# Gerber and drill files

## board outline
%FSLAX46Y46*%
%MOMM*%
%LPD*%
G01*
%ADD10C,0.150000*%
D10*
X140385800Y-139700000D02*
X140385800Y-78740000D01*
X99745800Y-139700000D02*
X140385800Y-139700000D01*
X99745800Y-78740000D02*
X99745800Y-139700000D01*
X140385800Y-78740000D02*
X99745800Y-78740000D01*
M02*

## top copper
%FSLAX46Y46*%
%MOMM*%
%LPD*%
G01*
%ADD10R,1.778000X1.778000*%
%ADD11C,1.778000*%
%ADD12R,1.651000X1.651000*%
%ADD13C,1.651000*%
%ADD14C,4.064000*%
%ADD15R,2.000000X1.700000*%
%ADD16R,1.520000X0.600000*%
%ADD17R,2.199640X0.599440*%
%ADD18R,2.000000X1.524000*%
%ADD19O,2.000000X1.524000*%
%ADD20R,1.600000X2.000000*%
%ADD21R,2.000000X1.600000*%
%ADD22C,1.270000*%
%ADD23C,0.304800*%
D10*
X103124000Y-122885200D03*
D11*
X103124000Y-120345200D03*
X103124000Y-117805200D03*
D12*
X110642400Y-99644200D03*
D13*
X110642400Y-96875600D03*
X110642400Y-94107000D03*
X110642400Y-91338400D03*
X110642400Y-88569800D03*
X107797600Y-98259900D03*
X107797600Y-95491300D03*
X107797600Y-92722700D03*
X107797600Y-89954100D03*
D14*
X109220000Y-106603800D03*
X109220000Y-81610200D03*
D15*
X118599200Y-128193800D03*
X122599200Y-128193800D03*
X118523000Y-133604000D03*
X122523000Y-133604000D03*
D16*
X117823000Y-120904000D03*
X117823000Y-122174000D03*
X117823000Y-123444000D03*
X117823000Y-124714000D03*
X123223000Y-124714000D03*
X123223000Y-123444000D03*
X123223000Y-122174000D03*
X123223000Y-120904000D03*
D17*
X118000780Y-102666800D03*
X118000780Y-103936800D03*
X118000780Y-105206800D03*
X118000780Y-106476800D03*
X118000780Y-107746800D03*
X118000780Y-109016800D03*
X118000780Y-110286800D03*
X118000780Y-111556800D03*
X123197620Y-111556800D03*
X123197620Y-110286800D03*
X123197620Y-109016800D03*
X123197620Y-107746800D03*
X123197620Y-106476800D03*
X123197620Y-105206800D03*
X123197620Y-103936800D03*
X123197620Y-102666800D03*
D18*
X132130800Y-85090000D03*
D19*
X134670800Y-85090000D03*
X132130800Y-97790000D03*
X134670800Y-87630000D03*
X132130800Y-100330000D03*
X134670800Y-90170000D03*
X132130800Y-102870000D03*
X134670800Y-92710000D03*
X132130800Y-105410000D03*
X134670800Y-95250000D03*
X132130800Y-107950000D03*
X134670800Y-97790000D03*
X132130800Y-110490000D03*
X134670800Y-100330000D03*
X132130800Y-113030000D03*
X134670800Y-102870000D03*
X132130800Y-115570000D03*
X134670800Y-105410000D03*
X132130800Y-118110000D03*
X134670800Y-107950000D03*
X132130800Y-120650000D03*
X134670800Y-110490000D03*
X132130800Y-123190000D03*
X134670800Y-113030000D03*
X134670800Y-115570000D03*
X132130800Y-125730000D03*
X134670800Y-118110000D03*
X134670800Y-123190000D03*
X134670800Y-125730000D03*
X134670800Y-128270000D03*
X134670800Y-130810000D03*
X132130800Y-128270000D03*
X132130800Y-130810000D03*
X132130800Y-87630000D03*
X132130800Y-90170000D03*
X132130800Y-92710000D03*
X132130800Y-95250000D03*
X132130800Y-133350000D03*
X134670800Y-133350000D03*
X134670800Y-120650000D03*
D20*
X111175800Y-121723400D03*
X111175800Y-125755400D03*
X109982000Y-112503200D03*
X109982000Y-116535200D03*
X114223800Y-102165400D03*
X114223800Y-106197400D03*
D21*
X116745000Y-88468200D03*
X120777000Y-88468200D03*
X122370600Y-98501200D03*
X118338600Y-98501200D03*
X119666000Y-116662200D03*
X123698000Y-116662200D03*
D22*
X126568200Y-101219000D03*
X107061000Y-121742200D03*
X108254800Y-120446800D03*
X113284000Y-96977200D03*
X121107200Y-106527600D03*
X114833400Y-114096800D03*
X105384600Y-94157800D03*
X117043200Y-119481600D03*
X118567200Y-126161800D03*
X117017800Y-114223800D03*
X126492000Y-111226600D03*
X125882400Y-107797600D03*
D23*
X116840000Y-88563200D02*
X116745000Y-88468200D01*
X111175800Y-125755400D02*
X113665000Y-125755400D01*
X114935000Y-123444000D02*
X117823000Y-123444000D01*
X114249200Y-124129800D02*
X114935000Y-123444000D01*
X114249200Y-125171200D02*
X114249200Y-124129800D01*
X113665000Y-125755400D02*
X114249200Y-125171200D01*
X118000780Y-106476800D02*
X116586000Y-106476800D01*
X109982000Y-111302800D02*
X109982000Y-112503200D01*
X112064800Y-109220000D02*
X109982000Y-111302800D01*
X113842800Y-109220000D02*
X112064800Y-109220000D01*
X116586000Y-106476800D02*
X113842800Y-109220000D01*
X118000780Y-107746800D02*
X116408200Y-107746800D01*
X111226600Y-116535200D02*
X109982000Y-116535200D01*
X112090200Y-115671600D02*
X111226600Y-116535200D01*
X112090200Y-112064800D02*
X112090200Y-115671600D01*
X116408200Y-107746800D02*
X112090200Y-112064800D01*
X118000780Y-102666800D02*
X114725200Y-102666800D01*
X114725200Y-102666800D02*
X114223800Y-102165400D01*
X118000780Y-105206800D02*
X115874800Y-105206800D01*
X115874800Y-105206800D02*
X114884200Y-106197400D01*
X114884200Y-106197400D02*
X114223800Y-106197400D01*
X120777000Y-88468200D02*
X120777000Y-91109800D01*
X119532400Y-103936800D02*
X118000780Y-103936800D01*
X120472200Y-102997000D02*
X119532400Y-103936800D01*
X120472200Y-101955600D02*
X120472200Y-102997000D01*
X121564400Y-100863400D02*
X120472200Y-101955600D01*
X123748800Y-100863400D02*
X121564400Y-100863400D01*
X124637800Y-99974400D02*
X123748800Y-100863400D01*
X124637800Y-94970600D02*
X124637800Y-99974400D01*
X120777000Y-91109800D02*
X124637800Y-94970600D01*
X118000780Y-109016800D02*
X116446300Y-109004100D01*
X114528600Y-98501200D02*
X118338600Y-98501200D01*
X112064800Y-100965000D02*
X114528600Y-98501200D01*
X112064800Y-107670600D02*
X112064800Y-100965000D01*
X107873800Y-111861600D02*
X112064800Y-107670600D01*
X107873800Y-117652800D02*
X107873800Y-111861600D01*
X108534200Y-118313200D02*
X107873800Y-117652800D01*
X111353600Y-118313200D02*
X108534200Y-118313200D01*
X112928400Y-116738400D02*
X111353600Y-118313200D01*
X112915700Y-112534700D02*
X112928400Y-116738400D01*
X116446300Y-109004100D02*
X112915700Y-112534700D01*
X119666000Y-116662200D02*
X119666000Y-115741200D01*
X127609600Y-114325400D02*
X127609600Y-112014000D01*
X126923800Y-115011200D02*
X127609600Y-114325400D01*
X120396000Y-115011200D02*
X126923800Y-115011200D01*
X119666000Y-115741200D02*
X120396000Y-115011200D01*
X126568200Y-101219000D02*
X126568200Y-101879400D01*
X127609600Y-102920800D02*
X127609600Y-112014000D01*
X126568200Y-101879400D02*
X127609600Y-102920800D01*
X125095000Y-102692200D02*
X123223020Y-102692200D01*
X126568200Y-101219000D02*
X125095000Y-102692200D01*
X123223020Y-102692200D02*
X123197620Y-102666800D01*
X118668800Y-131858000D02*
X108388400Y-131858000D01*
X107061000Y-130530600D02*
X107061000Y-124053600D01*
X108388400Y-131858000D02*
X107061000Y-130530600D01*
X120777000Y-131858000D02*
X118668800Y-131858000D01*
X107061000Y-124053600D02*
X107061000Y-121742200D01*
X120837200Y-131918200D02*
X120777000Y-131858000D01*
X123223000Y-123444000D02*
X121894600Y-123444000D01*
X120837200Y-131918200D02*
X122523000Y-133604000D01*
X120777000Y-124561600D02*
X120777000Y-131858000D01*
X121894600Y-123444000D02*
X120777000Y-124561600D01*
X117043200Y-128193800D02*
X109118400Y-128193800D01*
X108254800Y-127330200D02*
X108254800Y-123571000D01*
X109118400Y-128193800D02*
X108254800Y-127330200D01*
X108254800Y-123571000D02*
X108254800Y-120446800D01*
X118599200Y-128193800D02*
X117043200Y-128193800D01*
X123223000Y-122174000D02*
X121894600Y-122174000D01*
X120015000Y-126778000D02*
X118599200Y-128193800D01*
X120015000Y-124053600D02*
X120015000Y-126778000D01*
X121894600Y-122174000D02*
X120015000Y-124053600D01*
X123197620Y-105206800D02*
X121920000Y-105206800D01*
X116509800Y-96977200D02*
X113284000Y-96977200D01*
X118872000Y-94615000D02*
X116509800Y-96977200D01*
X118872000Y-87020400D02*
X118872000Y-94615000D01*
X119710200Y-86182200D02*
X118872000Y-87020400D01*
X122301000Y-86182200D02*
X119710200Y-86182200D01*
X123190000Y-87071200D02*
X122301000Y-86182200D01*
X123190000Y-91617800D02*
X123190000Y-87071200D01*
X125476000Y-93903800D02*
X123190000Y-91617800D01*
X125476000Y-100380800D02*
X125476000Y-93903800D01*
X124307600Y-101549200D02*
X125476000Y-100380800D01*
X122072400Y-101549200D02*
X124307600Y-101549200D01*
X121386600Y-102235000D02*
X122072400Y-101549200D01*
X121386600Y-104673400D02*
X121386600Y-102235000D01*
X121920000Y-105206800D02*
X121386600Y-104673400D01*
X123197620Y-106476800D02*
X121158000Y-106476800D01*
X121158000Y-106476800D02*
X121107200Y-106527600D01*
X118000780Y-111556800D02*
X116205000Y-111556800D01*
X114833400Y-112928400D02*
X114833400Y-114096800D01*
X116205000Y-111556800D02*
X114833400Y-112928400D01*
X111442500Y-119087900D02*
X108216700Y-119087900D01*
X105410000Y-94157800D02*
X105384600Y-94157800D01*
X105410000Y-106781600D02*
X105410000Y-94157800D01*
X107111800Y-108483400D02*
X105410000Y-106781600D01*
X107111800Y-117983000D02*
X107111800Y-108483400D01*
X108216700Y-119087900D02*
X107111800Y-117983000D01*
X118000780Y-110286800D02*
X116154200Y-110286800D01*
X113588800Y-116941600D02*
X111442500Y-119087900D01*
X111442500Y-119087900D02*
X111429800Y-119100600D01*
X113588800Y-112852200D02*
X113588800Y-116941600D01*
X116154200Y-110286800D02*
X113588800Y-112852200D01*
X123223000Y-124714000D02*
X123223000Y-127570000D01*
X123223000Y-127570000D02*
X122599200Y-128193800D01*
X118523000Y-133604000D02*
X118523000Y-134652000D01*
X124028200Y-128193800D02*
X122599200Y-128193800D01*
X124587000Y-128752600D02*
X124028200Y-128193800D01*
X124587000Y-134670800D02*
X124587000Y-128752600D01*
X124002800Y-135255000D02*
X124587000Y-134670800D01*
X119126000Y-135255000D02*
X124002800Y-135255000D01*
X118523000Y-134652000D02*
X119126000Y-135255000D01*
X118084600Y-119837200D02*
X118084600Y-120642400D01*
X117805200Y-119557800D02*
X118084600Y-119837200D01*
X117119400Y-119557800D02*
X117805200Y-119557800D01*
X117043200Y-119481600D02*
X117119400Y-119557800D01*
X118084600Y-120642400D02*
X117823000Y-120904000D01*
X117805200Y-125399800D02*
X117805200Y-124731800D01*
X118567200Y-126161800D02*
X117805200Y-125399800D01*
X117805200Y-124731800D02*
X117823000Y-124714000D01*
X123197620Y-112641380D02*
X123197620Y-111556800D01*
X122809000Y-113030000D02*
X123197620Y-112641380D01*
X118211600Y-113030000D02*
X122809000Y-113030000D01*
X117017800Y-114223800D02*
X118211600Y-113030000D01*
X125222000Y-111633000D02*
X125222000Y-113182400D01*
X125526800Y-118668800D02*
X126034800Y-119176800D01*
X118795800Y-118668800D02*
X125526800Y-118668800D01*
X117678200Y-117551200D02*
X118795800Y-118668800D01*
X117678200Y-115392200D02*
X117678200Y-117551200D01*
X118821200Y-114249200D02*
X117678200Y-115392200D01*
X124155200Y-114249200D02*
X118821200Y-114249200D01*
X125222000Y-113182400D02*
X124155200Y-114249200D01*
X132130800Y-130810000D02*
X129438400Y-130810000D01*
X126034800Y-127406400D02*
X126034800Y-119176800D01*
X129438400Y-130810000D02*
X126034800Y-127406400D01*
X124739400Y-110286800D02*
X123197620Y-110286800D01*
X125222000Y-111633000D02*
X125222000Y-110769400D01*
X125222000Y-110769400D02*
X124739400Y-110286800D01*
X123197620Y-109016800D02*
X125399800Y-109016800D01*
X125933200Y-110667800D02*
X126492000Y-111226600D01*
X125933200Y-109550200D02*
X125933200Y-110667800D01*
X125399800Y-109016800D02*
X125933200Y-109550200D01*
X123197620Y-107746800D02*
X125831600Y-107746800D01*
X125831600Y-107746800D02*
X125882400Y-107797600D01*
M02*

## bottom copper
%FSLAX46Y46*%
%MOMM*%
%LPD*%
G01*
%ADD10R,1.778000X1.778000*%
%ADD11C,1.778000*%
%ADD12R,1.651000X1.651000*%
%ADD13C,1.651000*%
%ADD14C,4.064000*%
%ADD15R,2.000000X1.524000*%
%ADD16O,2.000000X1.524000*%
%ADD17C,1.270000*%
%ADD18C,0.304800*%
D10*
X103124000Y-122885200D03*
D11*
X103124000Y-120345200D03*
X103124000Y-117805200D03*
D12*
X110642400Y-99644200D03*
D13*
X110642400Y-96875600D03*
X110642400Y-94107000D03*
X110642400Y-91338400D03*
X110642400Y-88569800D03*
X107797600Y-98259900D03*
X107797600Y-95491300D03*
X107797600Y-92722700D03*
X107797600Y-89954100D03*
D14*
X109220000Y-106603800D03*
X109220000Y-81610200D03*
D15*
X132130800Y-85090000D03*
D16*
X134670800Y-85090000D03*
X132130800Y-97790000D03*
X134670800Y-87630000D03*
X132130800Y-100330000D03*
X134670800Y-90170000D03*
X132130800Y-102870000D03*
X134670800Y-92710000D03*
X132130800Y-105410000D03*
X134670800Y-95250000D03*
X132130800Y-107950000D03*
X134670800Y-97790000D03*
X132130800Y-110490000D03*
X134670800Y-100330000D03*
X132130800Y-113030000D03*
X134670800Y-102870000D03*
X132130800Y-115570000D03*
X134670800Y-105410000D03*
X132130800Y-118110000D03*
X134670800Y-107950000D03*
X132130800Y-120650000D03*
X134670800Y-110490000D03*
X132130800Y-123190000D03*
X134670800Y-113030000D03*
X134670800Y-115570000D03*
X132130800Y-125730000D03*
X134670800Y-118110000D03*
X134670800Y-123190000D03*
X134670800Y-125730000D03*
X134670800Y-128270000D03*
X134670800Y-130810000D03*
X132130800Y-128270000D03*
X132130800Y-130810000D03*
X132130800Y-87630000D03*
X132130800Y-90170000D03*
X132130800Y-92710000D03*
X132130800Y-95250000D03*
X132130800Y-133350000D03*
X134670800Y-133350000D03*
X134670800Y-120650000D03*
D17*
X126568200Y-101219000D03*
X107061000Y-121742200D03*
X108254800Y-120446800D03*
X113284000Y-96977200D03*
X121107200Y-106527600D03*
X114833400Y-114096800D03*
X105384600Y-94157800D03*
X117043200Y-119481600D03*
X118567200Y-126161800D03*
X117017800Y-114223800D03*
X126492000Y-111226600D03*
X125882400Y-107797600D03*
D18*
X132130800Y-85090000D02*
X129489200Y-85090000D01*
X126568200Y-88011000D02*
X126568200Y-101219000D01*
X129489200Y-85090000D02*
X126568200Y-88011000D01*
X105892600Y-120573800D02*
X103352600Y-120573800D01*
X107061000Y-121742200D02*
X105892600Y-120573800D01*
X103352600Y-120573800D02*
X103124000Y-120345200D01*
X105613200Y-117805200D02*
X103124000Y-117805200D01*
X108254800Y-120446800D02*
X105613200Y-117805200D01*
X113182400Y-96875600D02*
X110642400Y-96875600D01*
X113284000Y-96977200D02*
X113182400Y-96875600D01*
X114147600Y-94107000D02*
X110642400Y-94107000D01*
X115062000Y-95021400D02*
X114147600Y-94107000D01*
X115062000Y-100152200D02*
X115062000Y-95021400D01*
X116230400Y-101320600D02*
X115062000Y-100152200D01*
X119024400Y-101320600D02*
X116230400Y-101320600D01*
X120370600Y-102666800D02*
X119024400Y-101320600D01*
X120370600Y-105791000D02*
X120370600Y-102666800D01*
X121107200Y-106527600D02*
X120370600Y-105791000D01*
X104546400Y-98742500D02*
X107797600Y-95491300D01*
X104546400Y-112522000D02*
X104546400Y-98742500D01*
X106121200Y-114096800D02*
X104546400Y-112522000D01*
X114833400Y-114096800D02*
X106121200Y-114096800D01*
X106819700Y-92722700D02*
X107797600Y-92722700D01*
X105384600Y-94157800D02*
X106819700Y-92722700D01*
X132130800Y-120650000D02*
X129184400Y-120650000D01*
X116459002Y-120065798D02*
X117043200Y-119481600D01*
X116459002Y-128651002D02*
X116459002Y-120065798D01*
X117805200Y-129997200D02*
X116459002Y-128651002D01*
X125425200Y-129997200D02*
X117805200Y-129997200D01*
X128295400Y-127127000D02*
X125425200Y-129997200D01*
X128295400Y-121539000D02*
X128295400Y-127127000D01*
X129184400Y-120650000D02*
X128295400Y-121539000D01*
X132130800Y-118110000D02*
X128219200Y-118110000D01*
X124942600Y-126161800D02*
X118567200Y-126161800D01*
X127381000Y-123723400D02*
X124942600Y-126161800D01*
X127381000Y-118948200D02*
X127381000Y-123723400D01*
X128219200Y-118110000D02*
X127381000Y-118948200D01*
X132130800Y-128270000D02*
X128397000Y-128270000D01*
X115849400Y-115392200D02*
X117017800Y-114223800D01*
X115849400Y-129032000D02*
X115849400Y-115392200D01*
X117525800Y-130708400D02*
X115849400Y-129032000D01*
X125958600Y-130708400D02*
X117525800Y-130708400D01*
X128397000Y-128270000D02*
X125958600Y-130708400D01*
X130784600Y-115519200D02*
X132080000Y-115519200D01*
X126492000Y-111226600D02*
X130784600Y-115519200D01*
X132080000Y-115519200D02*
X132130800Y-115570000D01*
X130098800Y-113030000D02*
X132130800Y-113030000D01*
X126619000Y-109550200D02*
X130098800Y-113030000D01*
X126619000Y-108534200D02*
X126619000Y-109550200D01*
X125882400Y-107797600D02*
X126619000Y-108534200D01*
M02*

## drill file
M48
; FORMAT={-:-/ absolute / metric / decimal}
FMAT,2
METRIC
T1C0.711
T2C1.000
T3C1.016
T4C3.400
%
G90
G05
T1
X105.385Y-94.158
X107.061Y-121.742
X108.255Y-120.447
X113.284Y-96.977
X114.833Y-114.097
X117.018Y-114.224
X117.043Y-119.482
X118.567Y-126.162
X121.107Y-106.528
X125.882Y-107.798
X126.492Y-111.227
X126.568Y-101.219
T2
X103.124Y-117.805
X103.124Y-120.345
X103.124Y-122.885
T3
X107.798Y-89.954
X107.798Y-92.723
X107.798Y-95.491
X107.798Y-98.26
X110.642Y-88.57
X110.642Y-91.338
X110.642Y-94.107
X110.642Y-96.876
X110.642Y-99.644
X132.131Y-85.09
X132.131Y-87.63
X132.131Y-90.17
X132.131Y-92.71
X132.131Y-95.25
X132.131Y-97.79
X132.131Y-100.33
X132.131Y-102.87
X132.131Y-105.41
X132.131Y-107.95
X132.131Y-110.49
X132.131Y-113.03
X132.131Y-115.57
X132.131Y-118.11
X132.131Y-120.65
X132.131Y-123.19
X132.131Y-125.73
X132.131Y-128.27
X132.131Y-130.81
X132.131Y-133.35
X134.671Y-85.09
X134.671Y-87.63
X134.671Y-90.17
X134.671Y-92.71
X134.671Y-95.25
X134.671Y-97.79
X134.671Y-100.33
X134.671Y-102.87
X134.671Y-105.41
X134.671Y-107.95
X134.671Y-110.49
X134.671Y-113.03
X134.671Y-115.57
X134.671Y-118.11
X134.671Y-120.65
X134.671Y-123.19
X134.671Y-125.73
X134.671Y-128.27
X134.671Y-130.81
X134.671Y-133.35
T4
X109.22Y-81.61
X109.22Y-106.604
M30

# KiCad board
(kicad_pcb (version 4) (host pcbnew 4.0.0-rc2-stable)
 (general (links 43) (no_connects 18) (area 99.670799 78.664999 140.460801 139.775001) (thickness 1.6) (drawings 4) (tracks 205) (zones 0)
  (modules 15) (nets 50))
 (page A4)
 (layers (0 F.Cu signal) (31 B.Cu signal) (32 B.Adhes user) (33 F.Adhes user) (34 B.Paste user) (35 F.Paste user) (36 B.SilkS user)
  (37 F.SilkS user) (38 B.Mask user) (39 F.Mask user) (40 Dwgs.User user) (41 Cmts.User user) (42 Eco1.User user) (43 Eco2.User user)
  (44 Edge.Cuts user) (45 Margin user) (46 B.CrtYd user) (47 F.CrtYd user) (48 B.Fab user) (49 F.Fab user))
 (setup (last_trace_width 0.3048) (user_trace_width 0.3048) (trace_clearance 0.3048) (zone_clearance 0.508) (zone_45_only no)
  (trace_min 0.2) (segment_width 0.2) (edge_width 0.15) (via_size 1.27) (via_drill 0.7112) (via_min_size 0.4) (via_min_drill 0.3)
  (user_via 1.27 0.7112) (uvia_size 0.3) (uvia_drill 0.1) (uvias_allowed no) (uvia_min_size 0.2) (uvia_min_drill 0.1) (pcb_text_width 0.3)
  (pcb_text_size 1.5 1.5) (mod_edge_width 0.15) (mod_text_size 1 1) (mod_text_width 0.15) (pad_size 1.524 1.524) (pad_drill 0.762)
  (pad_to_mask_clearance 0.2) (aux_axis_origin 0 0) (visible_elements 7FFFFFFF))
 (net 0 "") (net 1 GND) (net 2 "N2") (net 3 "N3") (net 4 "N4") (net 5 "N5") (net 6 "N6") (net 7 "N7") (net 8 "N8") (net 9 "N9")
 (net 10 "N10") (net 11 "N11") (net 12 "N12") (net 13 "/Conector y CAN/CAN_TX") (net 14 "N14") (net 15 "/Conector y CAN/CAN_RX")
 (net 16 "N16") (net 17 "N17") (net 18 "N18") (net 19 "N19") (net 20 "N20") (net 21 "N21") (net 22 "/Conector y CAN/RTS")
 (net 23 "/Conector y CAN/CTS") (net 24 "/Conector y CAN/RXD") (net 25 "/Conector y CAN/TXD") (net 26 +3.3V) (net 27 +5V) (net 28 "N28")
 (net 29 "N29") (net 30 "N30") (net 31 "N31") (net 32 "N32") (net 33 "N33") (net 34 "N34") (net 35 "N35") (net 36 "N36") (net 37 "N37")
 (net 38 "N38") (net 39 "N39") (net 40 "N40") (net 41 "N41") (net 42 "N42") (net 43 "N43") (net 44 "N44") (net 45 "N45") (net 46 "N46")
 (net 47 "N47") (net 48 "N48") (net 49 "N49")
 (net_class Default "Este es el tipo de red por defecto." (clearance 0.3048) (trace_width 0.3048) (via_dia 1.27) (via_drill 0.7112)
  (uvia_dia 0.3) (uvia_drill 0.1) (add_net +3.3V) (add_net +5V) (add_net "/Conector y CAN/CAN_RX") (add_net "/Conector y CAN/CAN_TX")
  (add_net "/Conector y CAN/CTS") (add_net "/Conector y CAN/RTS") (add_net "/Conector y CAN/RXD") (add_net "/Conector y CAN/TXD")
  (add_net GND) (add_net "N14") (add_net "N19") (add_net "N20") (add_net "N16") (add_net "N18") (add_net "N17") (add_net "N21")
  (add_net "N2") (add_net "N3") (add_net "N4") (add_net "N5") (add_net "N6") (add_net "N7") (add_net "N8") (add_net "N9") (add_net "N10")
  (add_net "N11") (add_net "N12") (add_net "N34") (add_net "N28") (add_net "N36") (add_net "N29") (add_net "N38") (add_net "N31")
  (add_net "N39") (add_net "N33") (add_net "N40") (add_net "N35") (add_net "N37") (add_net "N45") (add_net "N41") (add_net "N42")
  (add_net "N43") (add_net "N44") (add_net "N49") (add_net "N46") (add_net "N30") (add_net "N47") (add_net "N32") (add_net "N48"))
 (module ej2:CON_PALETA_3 (layer F.Cu) (at 103.124 120.3452 90)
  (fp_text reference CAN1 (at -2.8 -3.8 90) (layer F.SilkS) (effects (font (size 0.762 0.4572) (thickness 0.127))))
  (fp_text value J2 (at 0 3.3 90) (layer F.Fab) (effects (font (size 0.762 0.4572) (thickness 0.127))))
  (pad 1 thru_hole rect (at -2.54 0 90) (size 1.778 1.778) (drill 1) (layers *.Cu *.Mask) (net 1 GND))
  (pad 2 thru_hole circle (at 0 0 90) (size 1.778 1.778) (drill 1) (layers *.Cu *.Mask) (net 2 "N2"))
  (pad 3 thru_hole circle (at 2.54 0 90) (size 1.778 1.778) (drill 1) (layers *.Cu *.Mask) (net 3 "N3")))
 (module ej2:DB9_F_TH (layer F.Cu) (at 109.22 94.107 90)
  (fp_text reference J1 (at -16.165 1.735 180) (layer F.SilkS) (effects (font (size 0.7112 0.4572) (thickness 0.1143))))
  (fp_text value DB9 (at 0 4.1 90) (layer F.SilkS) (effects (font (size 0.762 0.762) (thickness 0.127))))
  (pad 1 thru_hole rect (at -5.5372 1.4224 90) (size 1.651 1.651) (drill 1.016) (layers *.Cu *.Mask) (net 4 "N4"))
  (pad 2 thru_hole circle (at -2.7686 1.4224 90) (size 1.651 1.651) (drill 1.016) (layers *.Cu *.Mask) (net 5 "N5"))
  (pad 3 thru_hole circle (at 0 1.4224 90) (size 1.651 1.651) (drill 1.016) (layers *.Cu *.Mask) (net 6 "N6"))
  (pad 4 thru_hole circle (at 2.7686 1.4224 90) (size 1.651 1.651) (drill 1.016) (layers *.Cu *.Mask) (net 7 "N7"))
  (pad 5 thru_hole circle (at 5.5372 1.4224 90) (size 1.651 1.651) (drill 1.016) (layers *.Cu *.Mask) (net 1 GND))
  (pad 6 thru_hole circle (at -4.1529 -1.4224 90) (size 1.651 1.651) (drill 1.016) (layers *.Cu *.Mask) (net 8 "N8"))
  (pad 7 thru_hole circle (at -1.3843 -1.4224 90) (size 1.651 1.651) (drill 1.016) (layers *.Cu *.Mask) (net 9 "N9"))
  (pad 8 thru_hole circle (at 1.3843 -1.4224 90) (size 1.651 1.651) (drill 1.016) (layers *.Cu *.Mask) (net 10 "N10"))
  (pad 9 thru_hole circle (at 4.1529 -1.4224 90) (size 1.651 1.651) (drill 1.016) (layers *.Cu *.Mask) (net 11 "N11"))
  (pad 10 thru_hole circle (at -12.4968 0 90) (size 4.064 4.064) (drill 3.4) (layers *.Cu *.Mask))
  (pad 11 thru_hole circle (at 12.4968 0 90) (size 4.064 4.064) (drill 3.4) (layers *.Cu *.Mask)))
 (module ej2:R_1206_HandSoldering (layer F.Cu) (at 120.5992 128.1938)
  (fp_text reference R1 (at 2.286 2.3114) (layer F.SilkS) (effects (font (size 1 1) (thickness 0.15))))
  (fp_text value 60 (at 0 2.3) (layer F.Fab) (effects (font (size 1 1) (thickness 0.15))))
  (pad 1 smd rect (at -2 0) (size 2 1.7) (layers F.Cu F.Paste F.Mask) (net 3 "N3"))
  (pad 2 smd rect (at 2 0) (size 2 1.7) (layers F.Cu F.Paste F.Mask) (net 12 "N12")))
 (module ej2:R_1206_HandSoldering (layer F.Cu) (at 120.523 133.604)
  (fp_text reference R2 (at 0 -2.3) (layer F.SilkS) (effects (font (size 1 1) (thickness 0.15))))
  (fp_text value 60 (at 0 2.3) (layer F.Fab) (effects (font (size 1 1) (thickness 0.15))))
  (pad 1 smd rect (at -2 0) (size 2 1.7) (layers F.Cu F.Paste F.Mask) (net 12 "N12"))
  (pad 2 smd rect (at 2 0) (size 2 1.7) (layers F.Cu F.Paste F.Mask) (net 2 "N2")))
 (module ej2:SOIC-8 (layer F.Cu) (at 120.523 122.809)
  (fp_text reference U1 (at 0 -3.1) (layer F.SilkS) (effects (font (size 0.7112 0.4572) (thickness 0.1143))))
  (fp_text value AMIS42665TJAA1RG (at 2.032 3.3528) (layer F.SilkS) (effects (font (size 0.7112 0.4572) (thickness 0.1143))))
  (pad 1 smd rect (at -2.7 -1.905 270) (size 0.6 1.52) (layers F.Cu F.Paste F.Mask) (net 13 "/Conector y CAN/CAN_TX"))
  (pad 2 smd rect (at -2.7 -0.635 270) (size 0.6 1.52) (layers F.Cu F.Paste F.Mask) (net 1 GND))
  (pad 3 smd rect (at -2.7 0.635 270) (size 0.6 1.52) (layers F.Cu F.Paste F.Mask) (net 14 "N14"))
  (pad 4 smd rect (at -2.7 1.905 270) (size 0.6 1.52) (layers F.Cu F.Paste F.Mask) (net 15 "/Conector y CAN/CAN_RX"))
  (pad 5 smd rect (at 2.7 1.905 270) (size 0.6 1.52) (layers F.Cu F.Paste F.Mask) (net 12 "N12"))
  (pad 6 smd rect (at 2.7 0.635 270) (size 0.6 1.52) (layers F.Cu F.Paste F.Mask) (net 2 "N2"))
  (pad 7 smd rect (at 2.7 -0.635 270) (size 0.6 1.52) (layers F.Cu F.Paste F.Mask) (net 3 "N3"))
  (pad 8 smd rect (at 2.7 -1.905 270) (size 0.6 1.52) (layers F.Cu F.Paste F.Mask) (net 1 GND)))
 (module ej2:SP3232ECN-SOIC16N (layer F.Cu) (at 120.5992 107.1118 270)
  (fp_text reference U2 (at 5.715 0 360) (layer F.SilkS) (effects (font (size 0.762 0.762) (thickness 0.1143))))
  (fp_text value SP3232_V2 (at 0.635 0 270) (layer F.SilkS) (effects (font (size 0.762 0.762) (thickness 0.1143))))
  (pad 1 smd rect (at -4.445 2.59842 270) (size 0.59944 2.19964) (layers F.Cu F.Paste F.Mask) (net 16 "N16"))
  (pad 2 smd rect (at -3.175 2.59842 270) (size 0.59944 2.19964) (layers F.Cu F.Paste F.Mask) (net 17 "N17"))
  (pad 3 smd rect (at -1.905 2.59842 270) (size 0.59944 2.19964) (layers F.Cu F.Paste F.Mask) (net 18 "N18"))
  (pad 4 smd rect (at -0.635 2.59842 270) (size 0.59944 2.19964) (layers F.Cu F.Paste F.Mask) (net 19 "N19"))
  (pad 5 smd rect (at 0.635 2.59842 270) (size 0.59944 2.19964) (layers F.Cu F.Paste F.Mask) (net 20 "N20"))
  (pad 6 smd rect (at 1.905 2.59842 270) (size 0.59944 2.19964) (layers F.Cu F.Paste F.Mask) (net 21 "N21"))
  (pad 7 smd rect (at 3.175 2.59842 270) (size 0.59944 2.19964) (layers F.Cu F.Paste F.Mask) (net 10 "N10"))
  (pad 8 smd rect (at 4.445 2.59842 270) (size 0.59944 2.19964) (layers F.Cu F.Paste F.Mask) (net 9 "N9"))
  (pad 9 smd rect (at 4.445 -2.59842 270) (size 0.59944 2.19964) (layers F.Cu F.Paste F.Mask) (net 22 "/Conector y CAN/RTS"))
  (pad 10 smd rect (at 3.175 -2.59842 270) (size 0.59944 2.19964) (layers F.Cu F.Paste F.Mask) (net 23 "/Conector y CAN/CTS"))
  (pad 11 smd rect (at 1.905 -2.59842 270) (size 0.59944 2.19964) (layers F.Cu F.Paste F.Mask) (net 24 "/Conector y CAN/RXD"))
  (pad 12 smd rect (at 0.635 -2.59842 270) (size 0.59944 2.19964) (layers F.Cu F.Paste F.Mask) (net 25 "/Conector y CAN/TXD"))
  (pad 13 smd rect (at -0.635 -2.59842 270) (size 0.59944 2.19964) (layers F.Cu F.Paste F.Mask) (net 6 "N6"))
  (pad 14 smd rect (at -1.905 -2.59842 270) (size 0.59944 2.19964) (layers F.Cu F.Paste F.Mask) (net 5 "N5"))
  (pad 15 smd rect (at -3.175 -2.59842 270) (size 0.59944 2.19964) (layers F.Cu F.Paste F.Mask) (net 1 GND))
  (pad 16 smd rect (at -4.445 -2.59842 270) (size 0.59944 2.19964) (layers F.Cu F.Paste F.Mask) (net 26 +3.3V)))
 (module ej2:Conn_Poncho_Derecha (layer F.Cu) (at 132.1308 85.09)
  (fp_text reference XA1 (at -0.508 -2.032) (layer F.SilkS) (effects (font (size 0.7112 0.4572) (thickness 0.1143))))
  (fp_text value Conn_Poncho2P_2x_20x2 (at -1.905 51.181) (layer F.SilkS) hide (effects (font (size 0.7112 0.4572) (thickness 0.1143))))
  (pad 1 thru_hole rect (at 0 0 270) (size 1.524 2) (drill 1.016) (layers *.Cu *.Mask) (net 26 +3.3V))
  (pad 2 thru_hole oval (at 2.54 0 270) (size 1.524 2) (drill 1.016) (layers *.Cu *.Mask) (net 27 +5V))
  (pad 11 thru_hole oval (at 0 12.7 270) (size 1.524 2) (drill 1.016) (layers *.Cu *.Mask) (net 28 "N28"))
  (pad 4 thru_hole oval (at 2.54 2.54 270) (size 1.524 2) (drill 1.016) (layers *.Cu *.Mask) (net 1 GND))
  (pad 13 thru_hole oval (at 0 15.24 270) (size 1.524 2) (drill 1.016) (layers *.Cu *.Mask) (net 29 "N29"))
  (pad 6 thru_hole oval (at 2.54 5.08 270) (size 1.524 2) (drill 1.016) (layers *.Cu *.Mask) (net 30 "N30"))
  (pad 15 thru_hole oval (at 0 17.78 270) (size 1.524 2) (drill 1.016) (layers *.Cu *.Mask) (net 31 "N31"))
  (pad 8 thru_hole oval (at 2.54 7.62 270) (size 1.524 2) (drill 1.016) (layers *.Cu *.Mask) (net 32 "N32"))
  (pad 17 thru_hole oval (at 0 20.32 270) (size 1.524 2) (drill 1.016) (layers *.Cu *.Mask) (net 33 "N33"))
  (pad 10 thru_hole oval (at 2.54 10.16 270) (size 1.524 2) (drill 1.016) (layers *.Cu *.Mask) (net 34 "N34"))
  (pad 19 thru_hole oval (at 0 22.86 270) (size 1.524 2) (drill 1.016) (layers *.Cu *.Mask) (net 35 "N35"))
  (pad 12 thru_hole oval (at 2.54 12.7 270) (size 1.524 2) (drill 1.016) (layers *.Cu *.Mask) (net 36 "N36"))
  (pad 21 thru_hole oval (at 0 25.4 270) (size 1.524 2) (drill 1.016) (layers *.Cu *.Mask) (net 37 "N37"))
  (pad 14 thru_hole oval (at 2.54 15.24 270) (size 1.524 2) (drill 1.016) (layers *.Cu *.Mask) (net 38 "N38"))
  (pad 23 thru_hole oval (at 0 27.94 270) (size 1.524 2) (drill 1.016) (layers *.Cu *.Mask) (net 25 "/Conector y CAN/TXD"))
  (pad 16 thru_hole oval (at 2.54 17.78 270) (size 1.524 2) (drill 1.016) (layers *.Cu *.Mask) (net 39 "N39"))
  (pad 25 thru_hole oval (at 0 30.48 270) (size 1.524 2) (drill 1.016) (layers *.Cu *.Mask) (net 24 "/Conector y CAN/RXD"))
  (pad 18 thru_hole oval (at 2.54 20.32 270) (size 1.524 2) (drill 1.016) (layers *.Cu *.Mask) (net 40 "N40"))
  (pad 27 thru_hole oval (at 0 33.02 270) (size 1.524 2) (drill 1.016) (layers *.Cu *.Mask) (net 15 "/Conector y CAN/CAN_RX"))
  (pad 20 thru_hole oval (at 2.54 22.86 270) (size 1.524 2) (drill 1.016) (layers *.Cu *.Mask) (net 1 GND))
  (pad 29 thru_hole oval (at 0 35.56 270) (size 1.524 2) (drill 1.016) (layers *.Cu *.Mask) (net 13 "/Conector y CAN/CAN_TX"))
  (pad 22 thru_hole oval (at 2.54 25.4 270) (size 1.524 2) (drill 1.016) (layers *.Cu *.Mask) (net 1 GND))
  (pad 31 thru_hole oval (at 0 38.1 270) (size 1.524 2) (drill 1.016) (layers *.Cu *.Mask) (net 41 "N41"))
  (pad 24 thru_hole oval (at 2.54 27.94 270) (size 1.524 2) (drill 1.016) (layers *.Cu *.Mask) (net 1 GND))
  (pad 26 thru_hole oval (at 2.54 30.48 270) (size 1.524 2) (drill 1.016) (layers *.Cu *.Mask) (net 1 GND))
  (pad 33 thru_hole oval (at 0 40.64 270) (size 1.524 2) (drill 1.016) (layers *.Cu *.Mask) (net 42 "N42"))
  (pad 28 thru_hole oval (at 2.54 33.02 270) (size 1.524 2) (drill 1.016) (layers *.Cu *.Mask) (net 1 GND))
  (pad 32 thru_hole oval (at 2.54 38.1 270) (size 1.524 2) (drill 1.016) (layers *.Cu *.Mask) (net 1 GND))
  (pad 34 thru_hole oval (at 2.54 40.64 270) (size 1.524 2) (drill 1.016) (layers *.Cu *.Mask) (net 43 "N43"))
  (pad 36 thru_hole oval (at 2.54 43.18 270) (size 1.524 2) (drill 1.016) (layers *.Cu *.Mask) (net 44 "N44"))
  (pad 38 thru_hole oval (at 2.54 45.72 270) (size 1.524 2) (drill 1.016) (layers *.Cu *.Mask) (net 1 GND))
  (pad 35 thru_hole oval (at 0 43.18 270) (size 1.524 2) (drill 1.016) (layers *.Cu *.Mask) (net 22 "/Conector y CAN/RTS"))
  (pad 37 thru_hole oval (at 0 45.72 270) (size 1.524 2) (drill 1.016) (layers *.Cu *.Mask) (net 23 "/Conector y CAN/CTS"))
  (pad 3 thru_hole oval (at 0 2.54 270) (size 1.524 2) (drill 1.016) (layers *.Cu *.Mask) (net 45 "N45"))
  (pad 5 thru_hole oval (at 0 5.08 270) (size 1.524 2) (drill 1.016) (layers *.Cu *.Mask) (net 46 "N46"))
  (pad 7 thru_hole oval (at 0 7.62 270) (size 1.524 2) (drill 1.016) (layers *.Cu *.Mask) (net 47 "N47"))
  (pad 9 thru_hole oval (at 0 10.16 270) (size 1.524 2) (drill 1.016) (layers *.Cu *.Mask) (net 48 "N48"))
  (pad 39 thru_hole oval (at 0 48.26 270) (size 1.524 2) (drill 1.016) (layers *.Cu *.Mask) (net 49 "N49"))
  (pad 40 thru_hole oval (at 2.54 48.26 270) (size 1.524 2) (drill 1.016) (layers *.Cu *.Mask) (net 1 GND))
  (pad 30 thru_hole oval (at 2.54 35.56 270) (size 1.524 2) (drill 1.016) (layers *.Cu *.Mask) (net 1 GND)))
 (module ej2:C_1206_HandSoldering (layer F.Cu) (at 111.1758 123.7234 270)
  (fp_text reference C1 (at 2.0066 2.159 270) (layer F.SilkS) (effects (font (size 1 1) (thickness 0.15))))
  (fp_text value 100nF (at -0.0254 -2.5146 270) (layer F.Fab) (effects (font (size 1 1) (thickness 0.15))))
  (pad 1 smd rect (at -2 0 270) (size 2 1.6) (layers F.Cu F.Paste F.Mask) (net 1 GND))
  (pad 2 smd rect (at 2.032 0 270) (size 2 1.6) (layers F.Cu F.Paste F.Mask) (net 14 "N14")))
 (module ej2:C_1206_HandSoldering (layer F.Cu) (at 109.982 114.5032 270)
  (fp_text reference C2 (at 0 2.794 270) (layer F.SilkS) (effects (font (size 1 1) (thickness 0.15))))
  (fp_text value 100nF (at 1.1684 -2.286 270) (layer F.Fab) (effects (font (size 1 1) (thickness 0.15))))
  (pad 1 smd rect (at -2 0 270) (size 2 1.6) (layers F.Cu F.Paste F.Mask) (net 19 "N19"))
  (pad 2 smd rect (at 2.032 0 270) (size 2 1.6) (layers F.Cu F.Paste F.Mask) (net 20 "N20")))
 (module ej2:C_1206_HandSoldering (layer F.Cu) (at 114.2238 104.1654 270)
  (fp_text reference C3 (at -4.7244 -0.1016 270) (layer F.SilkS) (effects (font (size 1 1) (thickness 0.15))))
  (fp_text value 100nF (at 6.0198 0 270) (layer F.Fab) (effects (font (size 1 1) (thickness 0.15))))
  (pad 1 smd rect (at -2 0 270) (size 2 1.6) (layers F.Cu F.Paste F.Mask) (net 16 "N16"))
  (pad 2 smd rect (at 2.032 0 270) (size 2 1.6) (layers F.Cu F.Paste F.Mask) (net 18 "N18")))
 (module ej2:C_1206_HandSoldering (layer F.Cu) (at 118.745 88.4682)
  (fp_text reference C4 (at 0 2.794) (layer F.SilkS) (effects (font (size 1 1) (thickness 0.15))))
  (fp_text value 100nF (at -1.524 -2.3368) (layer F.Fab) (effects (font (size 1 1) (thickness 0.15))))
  (pad 1 smd rect (at -2 0) (size 2 1.6) (layers F.Cu F.Paste F.Mask) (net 1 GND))
  (pad 2 smd rect (at 2.032 0) (size 2 1.6) (layers F.Cu F.Paste F.Mask) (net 17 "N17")))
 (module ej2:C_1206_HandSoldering (layer F.Cu) (at 120.3706 98.5012 180)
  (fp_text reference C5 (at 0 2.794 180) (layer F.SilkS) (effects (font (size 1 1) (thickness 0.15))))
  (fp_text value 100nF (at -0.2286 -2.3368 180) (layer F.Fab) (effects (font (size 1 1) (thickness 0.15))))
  (pad 1 smd rect (at -2 0 180) (size 2 1.6) (layers F.Cu F.Paste F.Mask) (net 1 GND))
  (pad 2 smd rect (at 2.032 0 180) (size 2 1.6) (layers F.Cu F.Paste F.Mask) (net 21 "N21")))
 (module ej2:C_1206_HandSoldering (layer F.Cu) (at 121.666 116.6622)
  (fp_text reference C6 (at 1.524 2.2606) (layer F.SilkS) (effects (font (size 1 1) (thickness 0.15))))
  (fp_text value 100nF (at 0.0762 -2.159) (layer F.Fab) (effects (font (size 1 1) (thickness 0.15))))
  (pad 1 smd rect (at -2 0) (size 2 1.6) (layers F.Cu F.Paste F.Mask) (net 26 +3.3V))
  (pad 2 smd rect (at 2.032 0) (size 2 1.6) (layers F.Cu F.Paste F.Mask) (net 1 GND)))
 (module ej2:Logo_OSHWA (layer F.Cu) (at 122.7582 82.8802)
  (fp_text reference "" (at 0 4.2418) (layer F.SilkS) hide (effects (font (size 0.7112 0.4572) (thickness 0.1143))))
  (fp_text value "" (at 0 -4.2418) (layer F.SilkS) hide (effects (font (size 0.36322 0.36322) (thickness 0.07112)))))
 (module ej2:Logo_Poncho (layer F.Cu) (at 106.6038 132.715)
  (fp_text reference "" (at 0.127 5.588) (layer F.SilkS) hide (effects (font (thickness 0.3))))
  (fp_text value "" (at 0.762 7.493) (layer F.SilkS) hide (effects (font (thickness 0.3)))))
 (gr_line (start 140.3858 139.7) (end 140.3858 78.74) (angle 90) (layer Edge.Cuts) (width 0.15))
 (gr_line (start 99.7458 139.7) (end 140.3858 139.7) (angle 90) (layer Edge.Cuts) (width 0.15))
 (gr_line (start 99.7458 78.74) (end 99.7458 139.7) (angle 90) (layer Edge.Cuts) (width 0.15))
 (gr_line (start 140.3858 78.74) (end 99.7458 78.74) (angle 90) (layer Edge.Cuts) (width 0.15))
 (segment (start 116.84 88.5632) (end 116.745 88.4682) (width 0.3048) (layer F.Cu) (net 1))
 (segment (start 111.1758 125.7554) (end 113.665 125.7554) (width 0.3048) (layer F.Cu) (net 14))
 (segment (start 114.935 123.444) (end 117.823 123.444) (width 0.3048) (layer F.Cu) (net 14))
 (segment (start 114.2492 124.1298) (end 114.935 123.444) (width 0.3048) (layer F.Cu) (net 14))
 (segment (start 114.2492 125.1712) (end 114.2492 124.1298) (width 0.3048) (layer F.Cu) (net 14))
 (segment (start 113.665 125.7554) (end 114.2492 125.1712) (width 0.3048) (layer F.Cu) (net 14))
 (segment (start 118.00078 106.4768) (end 116.586 106.4768) (width 0.3048) (layer F.Cu) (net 19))
 (segment (start 109.982 111.3028) (end 109.982 112.5032) (width 0.3048) (layer F.Cu) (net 19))
 (segment (start 112.0648 109.22) (end 109.982 111.3028) (width 0.3048) (layer F.Cu) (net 19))
 (segment (start 113.8428 109.22) (end 112.0648 109.22) (width 0.3048) (layer F.Cu) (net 19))
 (segment (start 116.586 106.4768) (end 113.8428 109.22) (width 0.3048) (layer F.Cu) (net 19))
 (segment (start 118.00078 107.7468) (end 116.4082 107.7468) (width 0.3048) (layer F.Cu) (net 20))
 (segment (start 111.2266 116.5352) (end 109.982 116.5352) (width 0.3048) (layer F.Cu) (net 20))
 (segment (start 112.0902 115.6716) (end 111.2266 116.5352) (width 0.3048) (layer F.Cu) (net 20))
 (segment (start 112.0902 112.0648) (end 112.0902 115.6716) (width 0.3048) (layer F.Cu) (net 20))
 (segment (start 116.4082 107.7468) (end 112.0902 112.0648) (width 0.3048) (layer F.Cu) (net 20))
 (segment (start 118.00078 102.6668) (end 114.7252 102.6668) (width 0.3048) (layer F.Cu) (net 16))
 (segment (start 114.7252 102.6668) (end 114.2238 102.1654) (width 0.3048) (layer F.Cu) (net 16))
 (segment (start 118.00078 105.2068) (end 115.8748 105.2068) (width 0.3048) (layer F.Cu) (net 18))
 (segment (start 115.8748 105.2068) (end 114.8842 106.1974) (width 0.3048) (layer F.Cu) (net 18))
 (segment (start 114.8842 106.1974) (end 114.2238 106.1974) (width 0.3048) (layer F.Cu) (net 18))
 (segment (start 120.777 88.4682) (end 120.777 91.1098) (width 0.3048) (layer F.Cu) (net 17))
 (segment (start 119.5324 103.9368) (end 118.00078 103.9368) (width 0.3048) (layer F.Cu) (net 17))
 (segment (start 120.4722 102.997) (end 119.5324 103.9368) (width 0.3048) (layer F.Cu) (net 17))
 (segment (start 120.4722 101.9556) (end 120.4722 102.997) (width 0.3048) (layer F.Cu) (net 17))
 (segment (start 121.5644 100.8634) (end 120.4722 101.9556) (width 0.3048) (layer F.Cu) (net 17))
 (segment (start 123.7488 100.8634) (end 121.5644 100.8634) (width 0.3048) (layer F.Cu) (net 17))
 (segment (start 124.6378 99.9744) (end 123.7488 100.8634) (width 0.3048) (layer F.Cu) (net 17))
 (segment (start 124.6378 94.9706) (end 124.6378 99.9744) (width 0.3048) (layer F.Cu) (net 17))
 (segment (start 120.777 91.1098) (end 124.6378 94.9706) (width 0.3048) (layer F.Cu) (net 17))
 (segment (start 118.00078 109.0168) (end 116.4463 109.0041) (width 0.3048) (layer F.Cu) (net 21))
 (segment (start 114.5286 98.5012) (end 118.3386 98.5012) (width 0.3048) (layer F.Cu) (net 21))
 (segment (start 112.0648 100.965) (end 114.5286 98.5012) (width 0.3048) (layer F.Cu) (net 21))
 (segment (start 112.0648 107.6706) (end 112.0648 100.965) (width 0.3048) (layer F.Cu) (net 21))
 (segment (start 107.8738 111.8616) (end 112.0648 107.6706) (width 0.3048) (layer F.Cu) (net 21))
 (segment (start 107.8738 117.6528) (end 107.8738 111.8616) (width 0.3048) (layer F.Cu) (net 21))
 (segment (start 108.5342 118.3132) (end 107.8738 117.6528) (width 0.3048) (layer F.Cu) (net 21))
 (segment (start 111.3536 118.3132) (end 108.5342 118.3132) (width 0.3048) (layer F.Cu) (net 21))
 (segment (start 112.9284 116.7384) (end 111.3536 118.3132) (width 0.3048) (layer F.Cu) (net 21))
 (segment (start 112.9157 112.5347) (end 112.9284 116.7384) (width 0.3048) (layer F.Cu) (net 21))
 (segment (start 116.4463 109.0041) (end 112.9157 112.5347) (width 0.3048) (layer F.Cu) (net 21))
 (segment (start 119.666 116.6622) (end 119.666 115.7412) (width 0.3048) (layer F.Cu) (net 26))
 (segment (start 127.6096 114.3254) (end 127.6096 112.014) (width 0.3048) (layer F.Cu) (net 26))
 (segment (start 126.9238 115.0112) (end 127.6096 114.3254) (width 0.3048) (layer F.Cu) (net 26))
 (segment (start 120.396 115.0112) (end 126.9238 115.0112) (width 0.3048) (layer F.Cu) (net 26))
 (segment (start 119.666 115.7412) (end 120.396 115.0112) (width 0.3048) (layer F.Cu) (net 26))
 (segment (start 126.5682 101.219) (end 126.5682 101.8794) (width 0.3048) (layer F.Cu) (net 26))
 (segment (start 127.6096 102.9208) (end 127.6096 112.014) (width 0.3048) (layer F.Cu) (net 26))
 (segment (start 126.5682 101.8794) (end 127.6096 102.9208) (width 0.3048) (layer F.Cu) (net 26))
 (segment (start 132.1308 85.09) (end 129.4892 85.09) (width 0.3048) (layer B.Cu) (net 26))
 (segment (start 125.095 102.6922) (end 123.22302 102.6922) (width 0.3048) (layer F.Cu) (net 26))
 (segment (start 126.5682 101.219) (end 125.095 102.6922) (width 0.3048) (layer F.Cu) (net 26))
 (via (at 126.5682 101.219) (size 1.27) (drill 0.7112) (layers F.Cu B.Cu) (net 26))
 (segment (start 126.5682 88.011) (end 126.5682 101.219) (width 0.3048) (layer B.Cu) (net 26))
 (segment (start 129.4892 85.09) (end 126.5682 88.011) (width 0.3048) (layer B.Cu) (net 26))
 (segment (start 123.22302 102.6922) (end 123.19762 102.6668) (width 0.3048) (layer F.Cu) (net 26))
 (segment (start 118.6688 131.858) (end 108.3884 131.858) (width 0.3048) (layer F.Cu) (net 2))
 (segment (start 107.061 130.5306) (end 107.061 124.0536) (width 0.3048) (layer F.Cu) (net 2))
 (segment (start 108.3884 131.858) (end 107.061 130.5306) (width 0.3048) (layer F.Cu) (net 2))
 (segment (start 120.777 131.858) (end 118.6688 131.858) (width 0.3048) (layer F.Cu) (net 2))
 (segment (start 105.8926 120.5738) (end 103.3526 120.5738) (width 0.3048) (layer B.Cu) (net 2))
 (segment (start 107.061 121.7422) (end 105.8926 120.5738) (width 0.3048) (layer B.Cu) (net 2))
 (via (at 107.061 121.7422) (size 1.27) (drill 0.7112) (layers F.Cu B.Cu) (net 2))
 (segment (start 107.061 124.0536) (end 107.061 121.7422) (width 0.3048) (layer F.Cu) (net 2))
 (segment (start 103.3526 120.5738) (end 103.124 120.3452) (width 0.3048) (layer B.Cu) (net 2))
 (segment (start 120.8372 131.9182) (end 120.777 131.858) (width 0.3048) (layer F.Cu) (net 2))
 (segment (start 123.223 123.444) (end 121.8946 123.444) (width 0.3048) (layer F.Cu) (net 2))
 (segment (start 120.8372 131.9182) (end 122.523 133.604) (width 0.3048) (layer F.Cu) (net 2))
 (segment (start 120.777 124.5616) (end 120.777 131.858) (width 0.3048) (layer F.Cu) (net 2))
 (segment (start 121.8946 123.444) (end 120.777 124.5616) (width 0.3048) (layer F.Cu) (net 2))
 (segment (start 117.0432 128.1938) (end 109.1184 128.1938) (width 0.3048) (layer F.Cu) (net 3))
 (segment (start 108.2548 127.3302) (end 108.2548 123.571) (width 0.3048) (layer F.Cu) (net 3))
 (segment (start 109.1184 128.1938) (end 108.2548 127.3302) (width 0.3048) (layer F.Cu) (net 3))
 (segment (start 108.2548 123.571) (end 108.2548 120.4468) (width 0.3048) (layer F.Cu) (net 3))
 (segment (start 118.5992 128.1938) (end 117.0432 128.1938) (width 0.3048) (layer F.Cu) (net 3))
 (segment (start 105.6132 117.8052) (end 103.124 117.8052) (width 0.3048) (layer B.Cu) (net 3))
 (segment (start 108.2548 120.4468) (end 105.6132 117.8052) (width 0.3048) (layer B.Cu) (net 3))
 (via (at 108.2548 120.4468) (size 1.27) (drill 0.7112) (layers F.Cu B.Cu) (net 3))
 (segment (start 123.223 122.174) (end 121.8946 122.174) (width 0.3048) (layer F.Cu) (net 3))
 (segment (start 120.015 126.778) (end 118.5992 128.1938) (width 0.3048) (layer F.Cu) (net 3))
 (segment (start 120.015 124.0536) (end 120.015 126.778) (width 0.3048) (layer F.Cu) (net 3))
 (segment (start 121.8946 122.174) (end 120.015 124.0536) (width 0.3048) (layer F.Cu) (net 3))
 (segment (start 123.19762 105.2068) (end 121.92 105.2068) (width 0.3048) (layer F.Cu) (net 5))
 (segment (start 113.1824 96.8756) (end 110.6424 96.8756) (width 0.3048) (layer B.Cu) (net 5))
 (segment (start 113.284 96.9772) (end 113.1824 96.8756) (width 0.3048) (layer B.Cu) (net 5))
 (via (at 113.284 96.9772) (size 1.27) (drill 0.7112) (layers F.Cu B.Cu) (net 5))
 (segment (start 116.5098 96.9772) (end 113.284 96.9772) (width 0.3048) (layer F.Cu) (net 5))
 (segment (start 118.872 94.615) (end 116.5098 96.9772) (width 0.3048) (layer F.Cu) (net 5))
 (segment (start 118.872 87.0204) (end 118.872 94.615) (width 0.3048) (layer F.Cu) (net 5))
 (segment (start 119.7102 86.1822) (end 118.872 87.0204) (width 0.3048) (layer F.Cu) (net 5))
 (segment (start 122.301 86.1822) (end 119.7102 86.1822) (width 0.3048) (layer F.Cu) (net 5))
 (segment (start 123.19 87.0712) (end 122.301 86.1822) (width 0.3048) (layer F.Cu) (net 5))
 (segment (start 123.19 91.6178) (end 123.19 87.0712) (width 0.3048) (layer F.Cu) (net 5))
 (segment (start 125.476 93.9038) (end 123.19 91.6178) (width 0.3048) (layer F.Cu) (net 5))
 (segment (start 125.476 100.3808) (end 125.476 93.9038) (width 0.3048) (layer F.Cu) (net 5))
 (segment (start 124.3076 101.5492) (end 125.476 100.3808) (width 0.3048) (layer F.Cu) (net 5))
 (segment (start 122.0724 101.5492) (end 124.3076 101.5492) (width 0.3048) (layer F.Cu) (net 5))
 (segment (start 121.3866 102.235) (end 122.0724 101.5492) (width 0.3048) (layer F.Cu) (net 5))
 (segment (start 121.3866 104.6734) (end 121.3866 102.235) (width 0.3048) (layer F.Cu) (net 5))
 (segment (start 121.92 105.2068) (end 121.3866 104.6734) (width 0.3048) (layer F.Cu) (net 5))
 (segment (start 123.19762 106.4768) (end 121.158 106.4768) (width 0.3048) (layer F.Cu) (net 6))
 (segment (start 114.1476 94.107) (end 110.6424 94.107) (width 0.3048) (layer B.Cu) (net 6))
 (segment (start 115.062 95.0214) (end 114.1476 94.107) (width 0.3048) (layer B.Cu) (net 6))
 (segment (start 115.062 100.1522) (end 115.062 95.0214) (width 0.3048) (layer B.Cu) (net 6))
 (segment (start 116.2304 101.3206) (end 115.062 100.1522) (width 0.3048) (layer B.Cu) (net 6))
 (segment (start 119.0244 101.3206) (end 116.2304 101.3206) (width 0.3048) (layer B.Cu) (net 6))
 (segment (start 120.3706 102.6668) (end 119.0244 101.3206) (width 0.3048) (layer B.Cu) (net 6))
 (segment (start 120.3706 105.791) (end 120.3706 102.6668) (width 0.3048) (layer B.Cu) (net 6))
 (segment (start 121.1072 106.5276) (end 120.3706 105.791) (width 0.3048) (layer B.Cu) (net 6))
 (via (at 121.1072 106.5276) (size 1.27) (drill 0.7112) (layers F.Cu B.Cu) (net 6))
 (segment (start 121.158 106.4768) (end 121.1072 106.5276) (width 0.3048) (layer F.Cu) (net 6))
 (segment (start 118.00078 111.5568) (end 116.205 111.5568) (width 0.3048) (layer F.Cu) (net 9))
 (segment (start 104.5464 98.7425) (end 107.7976 95.4913) (width 0.3048) (layer B.Cu) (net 9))
 (segment (start 104.5464 112.522) (end 104.5464 98.7425) (width 0.3048) (layer B.Cu) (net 9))
 (segment (start 106.1212 114.0968) (end 104.5464 112.522) (width 0.3048) (layer B.Cu) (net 9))
 (segment (start 114.8334 114.0968) (end 106.1212 114.0968) (width 0.3048) (layer B.Cu) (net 9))
 (via (at 114.8334 114.0968) (size 1.27) (drill 0.7112) (layers F.Cu B.Cu) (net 9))
 (segment (start 114.8334 112.9284) (end 114.8334 114.0968) (width 0.3048) (layer F.Cu) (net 9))
 (segment (start 116.205 111.5568) (end 114.8334 112.9284) (width 0.3048) (layer F.Cu) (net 9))
 (segment (start 111.4425 119.0879) (end 108.2167 119.0879) (width 0.3048) (layer F.Cu) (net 10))
 (segment (start 106.8197 92.7227) (end 107.7976 92.7227) (width 0.3048) (layer B.Cu) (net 10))
 (segment (start 105.3846 94.1578) (end 106.8197 92.7227) (width 0.3048) (layer B.Cu) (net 10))
 (via (at 105.3846 94.1578) (size 1.27) (drill 0.7112) (layers F.Cu B.Cu) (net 10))
 (segment (start 105.41 94.1578) (end 105.3846 94.1578) (width 0.3048) (layer F.Cu) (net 10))
 (segment (start 105.41 106.7816) (end 105.41 94.1578) (width 0.3048) (layer F.Cu) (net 10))
 (segment (start 107.1118 108.4834) (end 105.41 106.7816) (width 0.3048) (layer F.Cu) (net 10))
 (segment (start 107.1118 117.983) (end 107.1118 108.4834) (width 0.3048) (layer F.Cu) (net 10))
 (segment (start 108.2167 119.0879) (end 107.1118 117.983) (width 0.3048) (layer F.Cu) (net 10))
 (segment (start 118.00078 110.2868) (end 116.1542 110.2868) (width 0.3048) (layer F.Cu) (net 10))
 (segment (start 113.5888 116.9416) (end 111.4425 119.0879) (width 0.3048) (layer F.Cu) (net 10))
 (segment (start 111.4425 119.0879) (end 111.4298 119.1006) (width 0.3048) (layer F.Cu) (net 10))
 (segment (start 113.5888 112.8522) (end 113.5888 116.9416) (width 0.3048) (layer F.Cu) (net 10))
 (segment (start 116.1542 110.2868) (end 113.5888 112.8522) (width 0.3048) (layer F.Cu) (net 10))
 (segment (start 123.223 124.714) (end 123.223 127.57) (width 0.3048) (layer F.Cu) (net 12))
 (segment (start 123.223 127.57) (end 122.5992 128.1938) (width 0.3048) (layer F.Cu) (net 12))
 (segment (start 118.523 133.604) (end 118.523 134.652) (width 0.3048) (layer F.Cu) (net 12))
 (segment (start 124.0282 128.1938) (end 122.5992 128.1938) (width 0.3048) (layer F.Cu) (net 12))
 (segment (start 124.587 128.7526) (end 124.0282 128.1938) (width 0.3048) (layer F.Cu) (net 12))
 (segment (start 124.587 134.6708) (end 124.587 128.7526) (width 0.3048) (layer F.Cu) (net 12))
 (segment (start 124.0028 135.255) (end 124.587 134.6708) (width 0.3048) (layer F.Cu) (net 12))
 (segment (start 119.126 135.255) (end 124.0028 135.255) (width 0.3048) (layer F.Cu) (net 12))
 (segment (start 118.523 134.652) (end 119.126 135.255) (width 0.3048) (layer F.Cu) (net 12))
 (segment (start 132.1308 120.65) (end 129.1844 120.65) (width 0.3048) (layer B.Cu) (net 13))
 (segment (start 118.0846 119.8372) (end 118.0846 120.6424) (width 0.3048) (layer F.Cu) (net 13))
 (segment (start 117.8052 119.5578) (end 118.0846 119.8372) (width 0.3048) (layer F.Cu) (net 13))
 (segment (start 117.1194 119.5578) (end 117.8052 119.5578) (width 0.3048) (layer F.Cu) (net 13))
 (segment (start 117.0432 119.4816) (end 117.1194 119.5578) (width 0.3048) (layer F.Cu) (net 13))
 (via (at 117.0432 119.4816) (size 1.27) (drill 0.7112) (layers F.Cu B.Cu) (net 13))
 (segment (start 116.459002 120.065798) (end 117.0432 119.4816) (width 0.3048) (layer B.Cu) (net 13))
 (segment (start 116.459002 128.651002) (end 116.459002 120.065798) (width 0.3048) (layer B.Cu) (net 13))
 (segment (start 117.8052 129.9972) (end 116.459002 128.651002) (width 0.3048) (layer B.Cu) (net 13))
 (segment (start 125.4252 129.9972) (end 117.8052 129.9972) (width 0.3048) (layer B.Cu) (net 13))
 (segment (start 128.2954 127.127) (end 125.4252 129.9972) (width 0.3048) (layer B.Cu) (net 13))
 (segment (start 128.2954 121.539) (end 128.2954 127.127) (width 0.3048) (layer B.Cu) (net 13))
 (segment (start 129.1844 120.65) (end 128.2954 121.539) (width 0.3048) (layer B.Cu) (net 13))
 (segment (start 118.0846 120.6424) (end 117.823 120.904) (width 0.3048) (layer F.Cu) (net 13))
 (segment (start 132.1308 118.11) (end 128.2192 118.11) (width 0.3048) (layer B.Cu) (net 15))
 (segment (start 117.8052 125.3998) (end 117.8052 124.7318) (width 0.3048) (layer F.Cu) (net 15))
 (segment (start 118.5672 126.1618) (end 117.8052 125.3998) (width 0.3048) (layer F.Cu) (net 15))
 (via (at 118.5672 126.1618) (size 1.27) (drill 0.7112) (layers F.Cu B.Cu) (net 15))
 (segment (start 124.9426 126.1618) (end 118.5672 126.1618) (width 0.3048) (layer B.Cu) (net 15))
 (segment (start 127.381 123.7234) (end 124.9426 126.1618) (width 0.3048) (layer B.Cu) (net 15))
 (segment (start 127.381 118.9482) (end 127.381 123.7234) (width 0.3048) (layer B.Cu) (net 15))
 (segment (start 128.2192 118.11) (end 127.381 118.9482) (width 0.3048) (layer B.Cu) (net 15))
 (segment (start 117.8052 124.7318) (end 117.823 124.714) (width 0.3048) (layer F.Cu) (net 15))
 (segment (start 132.1308 128.27) (end 128.397 128.27) (width 0.3048) (layer B.Cu) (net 22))
 (segment (start 123.19762 112.64138) (end 123.19762 111.5568) (width 0.3048) (layer F.Cu) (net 22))
 (segment (start 122.809 113.03) (end 123.19762 112.64138) (width 0.3048) (layer F.Cu) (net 22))
 (segment (start 118.2116 113.03) (end 122.809 113.03) (width 0.3048) (layer F.Cu) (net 22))
 (segment (start 117.0178 114.2238) (end 118.2116 113.03) (width 0.3048) (layer F.Cu) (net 22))
 (via (at 117.0178 114.2238) (size 1.27) (drill 0.7112) (layers F.Cu B.Cu) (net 22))
 (segment (start 115.8494 115.3922) (end 117.0178 114.2238) (width 0.3048) (layer B.Cu) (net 22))
 (segment (start 115.8494 129.032) (end 115.8494 115.3922) (width 0.3048) (layer B.Cu) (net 22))
 (segment (start 117.5258 130.7084) (end 115.8494 129.032) (width 0.3048) (layer B.Cu) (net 22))
 (segment (start 125.9586 130.7084) (end 117.5258 130.7084) (width 0.3048) (layer B.Cu) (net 22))
 (segment (start 128.397 128.27) (end 125.9586 130.7084) (width 0.3048) (layer B.Cu) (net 22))
 (segment (start 125.222 111.633) (end 125.222 113.1824) (width 0.3048) (layer F.Cu) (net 23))
 (segment (start 125.5268 118.6688) (end 126.0348 119.1768) (width 0.3048) (layer F.Cu) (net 23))
 (segment (start 118.7958 118.6688) (end 125.5268 118.6688) (width 0.3048) (layer F.Cu) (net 23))
 (segment (start 117.6782 117.5512) (end 118.7958 118.6688) (width 0.3048) (layer F.Cu) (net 23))
 (segment (start 117.6782 115.3922) (end 117.6782 117.5512) (width 0.3048) (layer F.Cu) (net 23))
 (segment (start 118.8212 114.2492) (end 117.6782 115.3922) (width 0.3048) (layer F.Cu) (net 23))
 (segment (start 124.1552 114.2492) (end 118.8212 114.2492) (width 0.3048) (layer F.Cu) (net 23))
 (segment (start 125.222 113.1824) (end 124.1552 114.2492) (width 0.3048) (layer F.Cu) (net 23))
 (segment (start 132.1308 130.81) (end 129.4384 130.81) (width 0.3048) (layer F.Cu) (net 23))
 (segment (start 126.0348 127.4064) (end 126.0348 119.1768) (width 0.3048) (layer F.Cu) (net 23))
 (segment (start 129.4384 130.81) (end 126.0348 127.4064) (width 0.3048) (layer F.Cu) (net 23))
 (segment (start 124.7394 110.2868) (end 123.19762 110.2868) (width 0.3048) (layer F.Cu) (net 23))
 (segment (start 125.222 111.633) (end 125.222 110.7694) (width 0.3048) (layer F.Cu) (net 23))
 (segment (start 125.222 110.7694) (end 124.7394 110.2868) (width 0.3048) (layer F.Cu) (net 23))
 (segment (start 123.19762 109.0168) (end 125.3998 109.0168) (width 0.3048) (layer F.Cu) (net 24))
 (segment (start 130.7846 115.5192) (end 132.08 115.5192) (width 0.3048) (layer B.Cu) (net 24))
 (segment (start 126.492 111.2266) (end 130.7846 115.5192) (width 0.3048) (layer B.Cu) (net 24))
 (via (at 126.492 111.2266) (size 1.27) (drill 0.7112) (layers F.Cu B.Cu) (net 24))
 (segment (start 125.9332 110.6678) (end 126.492 111.2266) (width 0.3048) (layer F.Cu) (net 24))
 (segment (start 125.9332 109.5502) (end 125.9332 110.6678) (width 0.3048) (layer F.Cu) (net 24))
 (segment (start 125.3998 109.0168) (end 125.9332 109.5502) (width 0.3048) (layer F.Cu) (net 24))
 (segment (start 132.08 115.5192) (end 132.1308 115.57) (width 0.3048) (layer B.Cu) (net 24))
 (segment (start 123.19762 107.7468) (end 125.8316 107.7468) (width 0.3048) (layer F.Cu) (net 25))
 (segment (start 130.0988 113.03) (end 132.1308 113.03) (width 0.3048) (layer B.Cu) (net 25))
 (segment (start 126.619 109.5502) (end 130.0988 113.03) (width 0.3048) (layer B.Cu) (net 25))
 (segment (start 126.619 108.5342) (end 126.619 109.5502) (width 0.3048) (layer B.Cu) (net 25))
 (segment (start 125.8824 107.7976) (end 126.619 108.5342) (width 0.3048) (layer B.Cu) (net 25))
 (via (at 125.8824 107.7976) (size 1.27) (drill 0.7112) (layers F.Cu B.Cu) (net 25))
 (segment (start 125.8316 107.7468) (end 125.8824 107.7976) (width 0.3048) (layer F.Cu) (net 25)))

